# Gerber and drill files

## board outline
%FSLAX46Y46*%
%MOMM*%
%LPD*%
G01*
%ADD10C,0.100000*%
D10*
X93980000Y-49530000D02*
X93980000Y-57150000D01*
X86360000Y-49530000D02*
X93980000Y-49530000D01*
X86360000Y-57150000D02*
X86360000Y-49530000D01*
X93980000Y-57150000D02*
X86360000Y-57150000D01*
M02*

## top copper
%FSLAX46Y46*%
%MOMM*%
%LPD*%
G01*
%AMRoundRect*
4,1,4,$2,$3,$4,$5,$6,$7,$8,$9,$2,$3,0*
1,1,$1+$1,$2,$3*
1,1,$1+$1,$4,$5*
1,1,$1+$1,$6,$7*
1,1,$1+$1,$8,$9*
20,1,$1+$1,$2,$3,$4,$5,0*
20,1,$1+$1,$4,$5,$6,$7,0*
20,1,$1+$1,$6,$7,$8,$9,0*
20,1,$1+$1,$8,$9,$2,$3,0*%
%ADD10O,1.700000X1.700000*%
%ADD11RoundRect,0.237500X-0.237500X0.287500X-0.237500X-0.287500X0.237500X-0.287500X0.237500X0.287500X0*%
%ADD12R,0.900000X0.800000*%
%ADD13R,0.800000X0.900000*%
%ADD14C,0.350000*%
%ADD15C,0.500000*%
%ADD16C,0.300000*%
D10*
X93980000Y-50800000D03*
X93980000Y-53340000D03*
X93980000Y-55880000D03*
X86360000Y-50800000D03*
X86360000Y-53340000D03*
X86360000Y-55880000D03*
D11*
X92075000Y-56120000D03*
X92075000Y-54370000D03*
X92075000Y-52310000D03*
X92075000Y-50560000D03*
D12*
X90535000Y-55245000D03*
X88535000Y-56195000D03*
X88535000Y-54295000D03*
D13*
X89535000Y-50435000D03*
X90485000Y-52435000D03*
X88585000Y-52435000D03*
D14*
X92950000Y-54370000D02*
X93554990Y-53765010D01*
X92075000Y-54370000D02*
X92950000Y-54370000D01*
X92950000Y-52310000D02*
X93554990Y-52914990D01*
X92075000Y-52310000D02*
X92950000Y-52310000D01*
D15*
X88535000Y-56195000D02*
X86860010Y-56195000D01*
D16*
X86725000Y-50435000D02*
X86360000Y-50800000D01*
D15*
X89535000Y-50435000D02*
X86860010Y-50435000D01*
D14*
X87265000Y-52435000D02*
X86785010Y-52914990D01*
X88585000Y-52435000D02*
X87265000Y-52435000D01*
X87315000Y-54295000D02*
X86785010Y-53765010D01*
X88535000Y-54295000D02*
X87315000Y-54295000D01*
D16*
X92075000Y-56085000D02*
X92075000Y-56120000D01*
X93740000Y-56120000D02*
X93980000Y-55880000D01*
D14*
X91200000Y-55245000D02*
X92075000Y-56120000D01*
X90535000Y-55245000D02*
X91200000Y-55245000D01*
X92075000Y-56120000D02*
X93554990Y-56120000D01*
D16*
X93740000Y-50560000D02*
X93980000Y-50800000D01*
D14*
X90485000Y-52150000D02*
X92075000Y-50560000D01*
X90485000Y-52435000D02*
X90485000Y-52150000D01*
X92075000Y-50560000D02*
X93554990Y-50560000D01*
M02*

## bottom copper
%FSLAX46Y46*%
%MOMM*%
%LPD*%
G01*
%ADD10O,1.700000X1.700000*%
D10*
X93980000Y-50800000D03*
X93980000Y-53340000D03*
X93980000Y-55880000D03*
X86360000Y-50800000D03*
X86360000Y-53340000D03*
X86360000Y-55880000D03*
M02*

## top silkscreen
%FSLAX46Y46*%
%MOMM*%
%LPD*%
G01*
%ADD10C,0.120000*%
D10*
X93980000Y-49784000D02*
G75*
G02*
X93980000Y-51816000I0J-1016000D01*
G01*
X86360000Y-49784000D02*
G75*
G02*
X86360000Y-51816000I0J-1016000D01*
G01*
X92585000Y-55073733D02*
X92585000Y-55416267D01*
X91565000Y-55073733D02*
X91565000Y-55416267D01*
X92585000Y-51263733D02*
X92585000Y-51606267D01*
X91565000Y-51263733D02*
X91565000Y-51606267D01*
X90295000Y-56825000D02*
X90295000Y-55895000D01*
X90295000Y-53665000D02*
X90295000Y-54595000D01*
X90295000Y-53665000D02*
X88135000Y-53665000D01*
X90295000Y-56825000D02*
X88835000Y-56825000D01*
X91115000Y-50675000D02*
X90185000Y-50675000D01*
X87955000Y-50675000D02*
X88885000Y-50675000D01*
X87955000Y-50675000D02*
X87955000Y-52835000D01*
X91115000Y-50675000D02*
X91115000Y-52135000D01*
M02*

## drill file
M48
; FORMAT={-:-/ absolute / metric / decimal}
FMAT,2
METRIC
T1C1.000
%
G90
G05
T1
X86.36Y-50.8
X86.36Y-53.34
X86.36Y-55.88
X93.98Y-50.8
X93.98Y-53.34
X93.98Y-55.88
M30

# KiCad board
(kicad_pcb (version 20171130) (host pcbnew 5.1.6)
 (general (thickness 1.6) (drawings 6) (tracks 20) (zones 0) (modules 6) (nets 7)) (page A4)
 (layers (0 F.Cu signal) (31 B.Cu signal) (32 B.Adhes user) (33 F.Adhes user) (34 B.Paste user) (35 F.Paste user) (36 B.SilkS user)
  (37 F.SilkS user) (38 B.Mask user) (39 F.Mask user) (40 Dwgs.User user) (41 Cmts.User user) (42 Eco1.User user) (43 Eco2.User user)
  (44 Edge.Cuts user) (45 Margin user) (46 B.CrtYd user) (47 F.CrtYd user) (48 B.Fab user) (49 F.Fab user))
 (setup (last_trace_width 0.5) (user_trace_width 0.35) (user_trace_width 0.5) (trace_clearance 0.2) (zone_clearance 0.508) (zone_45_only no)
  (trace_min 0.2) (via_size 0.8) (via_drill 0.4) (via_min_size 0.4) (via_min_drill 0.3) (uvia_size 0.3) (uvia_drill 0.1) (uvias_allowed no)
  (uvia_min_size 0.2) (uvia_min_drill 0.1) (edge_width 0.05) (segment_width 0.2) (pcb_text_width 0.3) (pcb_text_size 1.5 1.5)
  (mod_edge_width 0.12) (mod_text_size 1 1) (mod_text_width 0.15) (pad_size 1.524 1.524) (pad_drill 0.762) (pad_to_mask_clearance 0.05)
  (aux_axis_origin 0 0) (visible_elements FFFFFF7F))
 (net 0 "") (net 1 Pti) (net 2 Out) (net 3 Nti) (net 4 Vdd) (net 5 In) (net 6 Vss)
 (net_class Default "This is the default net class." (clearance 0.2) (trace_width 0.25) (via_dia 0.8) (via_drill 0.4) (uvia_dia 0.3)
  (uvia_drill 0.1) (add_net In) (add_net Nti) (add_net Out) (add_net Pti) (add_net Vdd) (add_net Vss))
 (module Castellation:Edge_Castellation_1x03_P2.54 (layer F.Cu) (at 93.98 50.8)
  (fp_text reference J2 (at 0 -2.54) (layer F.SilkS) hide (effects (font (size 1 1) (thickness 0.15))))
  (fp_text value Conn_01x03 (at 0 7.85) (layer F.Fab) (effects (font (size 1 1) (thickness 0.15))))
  (fp_arc (start 0 0) (end 0 1.016) (angle -180) (layer F.SilkS) (width 0.12))
  (pad 1 thru_hole oval (at 0 0) (size 1.7 1.7) (drill 1) (layers *.Cu *.Mask) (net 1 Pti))
  (pad 2 thru_hole oval (at 0 2.54) (size 1.7 1.7) (drill 1) (layers *.Cu *.Mask) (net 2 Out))
  (pad 3 thru_hole oval (at 0 5.08) (size 1.7 1.7) (drill 1) (layers *.Cu *.Mask) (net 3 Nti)))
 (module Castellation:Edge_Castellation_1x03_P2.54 (layer F.Cu) (at 86.36 50.8)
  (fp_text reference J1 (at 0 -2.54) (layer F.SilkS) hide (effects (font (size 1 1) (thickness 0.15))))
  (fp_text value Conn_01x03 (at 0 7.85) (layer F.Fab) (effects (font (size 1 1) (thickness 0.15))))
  (fp_arc (start 0 0) (end 0 1.016) (angle -180) (layer F.SilkS) (width 0.12))
  (pad 1 thru_hole oval (at 0 0) (size 1.7 1.7) (drill 1) (layers *.Cu *.Mask) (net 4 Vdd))
  (pad 2 thru_hole oval (at 0 2.54) (size 1.7 1.7) (drill 1) (layers *.Cu *.Mask) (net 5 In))
  (pad 3 thru_hole oval (at 0 5.08) (size 1.7 1.7) (drill 1) (layers *.Cu *.Mask) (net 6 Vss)))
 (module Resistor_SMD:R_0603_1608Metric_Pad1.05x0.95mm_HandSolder (layer F.Cu) (at 92.075 55.245 270)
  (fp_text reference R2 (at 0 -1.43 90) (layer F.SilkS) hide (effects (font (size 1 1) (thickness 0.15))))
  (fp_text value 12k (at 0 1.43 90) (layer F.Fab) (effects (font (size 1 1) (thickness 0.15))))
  (fp_line (start -0.171267 -0.51) (end 0.171267 -0.51) (layer F.SilkS) (width 0.12))
  (fp_line (start -0.171267 0.51) (end 0.171267 0.51) (layer F.SilkS) (width 0.12))
  (pad 2 smd roundrect (at 0.875 0 270) (size 1.05 0.95) (layers F.Cu F.Paste F.Mask) (roundrect_rratio 0.25) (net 3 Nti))
  (pad 1 smd roundrect (at -0.875 0 270) (size 1.05 0.95) (layers F.Cu F.Paste F.Mask) (roundrect_rratio 0.25) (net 2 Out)))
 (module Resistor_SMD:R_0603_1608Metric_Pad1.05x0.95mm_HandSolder (layer F.Cu) (at 92.075 51.435 270)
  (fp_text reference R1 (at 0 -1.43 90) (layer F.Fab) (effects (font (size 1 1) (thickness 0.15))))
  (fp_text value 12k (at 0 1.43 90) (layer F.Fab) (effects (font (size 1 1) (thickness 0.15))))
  (fp_line (start -0.171267 -0.51) (end 0.171267 -0.51) (layer F.SilkS) (width 0.12))
  (fp_line (start -0.171267 0.51) (end 0.171267 0.51) (layer F.SilkS) (width 0.12))
  (pad 2 smd roundrect (at 0.875 0 270) (size 1.05 0.95) (layers F.Cu F.Paste F.Mask) (roundrect_rratio 0.25) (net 2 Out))
  (pad 1 smd roundrect (at -0.875 0 270) (size 1.05 0.95) (layers F.Cu F.Paste F.Mask) (roundrect_rratio 0.25) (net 1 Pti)))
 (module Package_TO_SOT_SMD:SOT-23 (layer F.Cu) (at 89.535 55.245)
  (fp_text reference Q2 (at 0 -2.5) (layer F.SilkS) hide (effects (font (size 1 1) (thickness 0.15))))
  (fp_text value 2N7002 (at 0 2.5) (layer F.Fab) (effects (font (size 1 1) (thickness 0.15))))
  (fp_line (start 0.76 1.58) (end 0.76 0.65) (layer F.SilkS) (width 0.12))
  (fp_line (start 0.76 -1.58) (end 0.76 -0.65) (layer F.SilkS) (width 0.12))
  (fp_line (start 0.76 -1.58) (end -1.4 -1.58) (layer F.SilkS) (width 0.12))
  (fp_line (start 0.76 1.58) (end -0.7 1.58) (layer F.SilkS) (width 0.12))
  (pad 3 smd rect (at 1 0) (size 0.9 0.8) (layers F.Cu F.Paste F.Mask) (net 3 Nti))
  (pad 2 smd rect (at -1 0.95) (size 0.9 0.8) (layers F.Cu F.Paste F.Mask) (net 6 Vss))
  (pad 1 smd rect (at -1 -0.95) (size 0.9 0.8) (layers F.Cu F.Paste F.Mask) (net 5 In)))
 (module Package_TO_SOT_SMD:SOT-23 (layer F.Cu) (at 89.535 51.435 90)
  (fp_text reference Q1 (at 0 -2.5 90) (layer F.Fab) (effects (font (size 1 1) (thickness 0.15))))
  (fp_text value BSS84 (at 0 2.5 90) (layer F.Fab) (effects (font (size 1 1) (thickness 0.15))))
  (fp_line (start 0.76 1.58) (end 0.76 0.65) (layer F.SilkS) (width 0.12))
  (fp_line (start 0.76 -1.58) (end 0.76 -0.65) (layer F.SilkS) (width 0.12))
  (fp_line (start 0.76 -1.58) (end -1.4 -1.58) (layer F.SilkS) (width 0.12))
  (fp_line (start 0.76 1.58) (end -0.7 1.58) (layer F.SilkS) (width 0.12))
  (pad 3 smd rect (at 1 0 90) (size 0.9 0.8) (layers F.Cu F.Paste F.Mask) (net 4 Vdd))
  (pad 2 smd rect (at -1 0.95 90) (size 0.9 0.8) (layers F.Cu F.Paste F.Mask) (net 1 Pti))
  (pad 1 smd rect (at -1 -0.95 90) (size 0.9 0.8) (layers F.Cu F.Paste F.Mask) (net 5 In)))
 (gr_line (start 93.98 49.53) (end 93.98 57.15) (layer Edge.Cuts) (width 0.1))
 (gr_line (start 86.36 49.53) (end 93.98 49.53) (layer Edge.Cuts) (width 0.1))
 (gr_line (start 86.36 57.15) (end 86.36 49.53) (layer Edge.Cuts) (width 0.1))
 (gr_line (start 93.98 57.15) (end 86.36 57.15) (layer Edge.Cuts) (width 0.1))
 (segment (start 92.95 54.37) (end 93.55499 53.76501) (width 0.35) (layer F.Cu) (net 2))
 (segment (start 92.075 54.37) (end 92.95 54.37) (width 0.35) (layer F.Cu) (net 2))
 (segment (start 92.95 52.31) (end 93.55499 52.91499) (width 0.35) (layer F.Cu) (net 2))
 (segment (start 92.075 52.31) (end 92.95 52.31) (width 0.35) (layer F.Cu) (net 2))
 (segment (start 88.535 56.195) (end 86.86001 56.195) (width 0.5) (layer F.Cu) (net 6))
 (segment (start 86.725 50.435) (end 86.36 50.8) (width 0.3) (layer F.Cu) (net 4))
 (segment (start 89.535 50.435) (end 86.86001 50.435) (width 0.5) (layer F.Cu) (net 4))
 (segment (start 87.265 52.435) (end 86.78501 52.91499) (width 0.35) (layer F.Cu) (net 5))
 (segment (start 88.585 52.435) (end 87.265 52.435) (width 0.35) (layer F.Cu) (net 5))
 (segment (start 87.315 54.295) (end 86.78501 53.76501) (width 0.35) (layer F.Cu) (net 5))
 (segment (start 88.535 54.295) (end 87.315 54.295) (width 0.35) (layer F.Cu) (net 5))
 (segment (start 92.075 56.085) (end 92.075 56.12) (width 0.3) (layer F.Cu) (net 3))
 (segment (start 93.74 56.12) (end 93.98 55.88) (width 0.3) (layer F.Cu) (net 3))
 (segment (start 91.2 55.245) (end 92.075 56.12) (width 0.35) (layer F.Cu) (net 3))
 (segment (start 90.535 55.245) (end 91.2 55.245) (width 0.35) (layer F.Cu) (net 3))
 (segment (start 92.075 56.12) (end 93.55499 56.12) (width 0.35) (layer F.Cu) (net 3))
 (segment (start 93.74 50.56) (end 93.98 50.8) (width 0.3) (layer F.Cu) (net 1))
 (segment (start 90.485 52.15) (end 92.075 50.56) (width 0.35) (layer F.Cu) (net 1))
 (segment (start 90.485 52.435) (end 90.485 52.15) (width 0.35) (layer F.Cu) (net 1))
 (segment (start 92.075 50.56) (end 93.55499 50.56) (width 0.35) (layer F.Cu) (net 1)))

